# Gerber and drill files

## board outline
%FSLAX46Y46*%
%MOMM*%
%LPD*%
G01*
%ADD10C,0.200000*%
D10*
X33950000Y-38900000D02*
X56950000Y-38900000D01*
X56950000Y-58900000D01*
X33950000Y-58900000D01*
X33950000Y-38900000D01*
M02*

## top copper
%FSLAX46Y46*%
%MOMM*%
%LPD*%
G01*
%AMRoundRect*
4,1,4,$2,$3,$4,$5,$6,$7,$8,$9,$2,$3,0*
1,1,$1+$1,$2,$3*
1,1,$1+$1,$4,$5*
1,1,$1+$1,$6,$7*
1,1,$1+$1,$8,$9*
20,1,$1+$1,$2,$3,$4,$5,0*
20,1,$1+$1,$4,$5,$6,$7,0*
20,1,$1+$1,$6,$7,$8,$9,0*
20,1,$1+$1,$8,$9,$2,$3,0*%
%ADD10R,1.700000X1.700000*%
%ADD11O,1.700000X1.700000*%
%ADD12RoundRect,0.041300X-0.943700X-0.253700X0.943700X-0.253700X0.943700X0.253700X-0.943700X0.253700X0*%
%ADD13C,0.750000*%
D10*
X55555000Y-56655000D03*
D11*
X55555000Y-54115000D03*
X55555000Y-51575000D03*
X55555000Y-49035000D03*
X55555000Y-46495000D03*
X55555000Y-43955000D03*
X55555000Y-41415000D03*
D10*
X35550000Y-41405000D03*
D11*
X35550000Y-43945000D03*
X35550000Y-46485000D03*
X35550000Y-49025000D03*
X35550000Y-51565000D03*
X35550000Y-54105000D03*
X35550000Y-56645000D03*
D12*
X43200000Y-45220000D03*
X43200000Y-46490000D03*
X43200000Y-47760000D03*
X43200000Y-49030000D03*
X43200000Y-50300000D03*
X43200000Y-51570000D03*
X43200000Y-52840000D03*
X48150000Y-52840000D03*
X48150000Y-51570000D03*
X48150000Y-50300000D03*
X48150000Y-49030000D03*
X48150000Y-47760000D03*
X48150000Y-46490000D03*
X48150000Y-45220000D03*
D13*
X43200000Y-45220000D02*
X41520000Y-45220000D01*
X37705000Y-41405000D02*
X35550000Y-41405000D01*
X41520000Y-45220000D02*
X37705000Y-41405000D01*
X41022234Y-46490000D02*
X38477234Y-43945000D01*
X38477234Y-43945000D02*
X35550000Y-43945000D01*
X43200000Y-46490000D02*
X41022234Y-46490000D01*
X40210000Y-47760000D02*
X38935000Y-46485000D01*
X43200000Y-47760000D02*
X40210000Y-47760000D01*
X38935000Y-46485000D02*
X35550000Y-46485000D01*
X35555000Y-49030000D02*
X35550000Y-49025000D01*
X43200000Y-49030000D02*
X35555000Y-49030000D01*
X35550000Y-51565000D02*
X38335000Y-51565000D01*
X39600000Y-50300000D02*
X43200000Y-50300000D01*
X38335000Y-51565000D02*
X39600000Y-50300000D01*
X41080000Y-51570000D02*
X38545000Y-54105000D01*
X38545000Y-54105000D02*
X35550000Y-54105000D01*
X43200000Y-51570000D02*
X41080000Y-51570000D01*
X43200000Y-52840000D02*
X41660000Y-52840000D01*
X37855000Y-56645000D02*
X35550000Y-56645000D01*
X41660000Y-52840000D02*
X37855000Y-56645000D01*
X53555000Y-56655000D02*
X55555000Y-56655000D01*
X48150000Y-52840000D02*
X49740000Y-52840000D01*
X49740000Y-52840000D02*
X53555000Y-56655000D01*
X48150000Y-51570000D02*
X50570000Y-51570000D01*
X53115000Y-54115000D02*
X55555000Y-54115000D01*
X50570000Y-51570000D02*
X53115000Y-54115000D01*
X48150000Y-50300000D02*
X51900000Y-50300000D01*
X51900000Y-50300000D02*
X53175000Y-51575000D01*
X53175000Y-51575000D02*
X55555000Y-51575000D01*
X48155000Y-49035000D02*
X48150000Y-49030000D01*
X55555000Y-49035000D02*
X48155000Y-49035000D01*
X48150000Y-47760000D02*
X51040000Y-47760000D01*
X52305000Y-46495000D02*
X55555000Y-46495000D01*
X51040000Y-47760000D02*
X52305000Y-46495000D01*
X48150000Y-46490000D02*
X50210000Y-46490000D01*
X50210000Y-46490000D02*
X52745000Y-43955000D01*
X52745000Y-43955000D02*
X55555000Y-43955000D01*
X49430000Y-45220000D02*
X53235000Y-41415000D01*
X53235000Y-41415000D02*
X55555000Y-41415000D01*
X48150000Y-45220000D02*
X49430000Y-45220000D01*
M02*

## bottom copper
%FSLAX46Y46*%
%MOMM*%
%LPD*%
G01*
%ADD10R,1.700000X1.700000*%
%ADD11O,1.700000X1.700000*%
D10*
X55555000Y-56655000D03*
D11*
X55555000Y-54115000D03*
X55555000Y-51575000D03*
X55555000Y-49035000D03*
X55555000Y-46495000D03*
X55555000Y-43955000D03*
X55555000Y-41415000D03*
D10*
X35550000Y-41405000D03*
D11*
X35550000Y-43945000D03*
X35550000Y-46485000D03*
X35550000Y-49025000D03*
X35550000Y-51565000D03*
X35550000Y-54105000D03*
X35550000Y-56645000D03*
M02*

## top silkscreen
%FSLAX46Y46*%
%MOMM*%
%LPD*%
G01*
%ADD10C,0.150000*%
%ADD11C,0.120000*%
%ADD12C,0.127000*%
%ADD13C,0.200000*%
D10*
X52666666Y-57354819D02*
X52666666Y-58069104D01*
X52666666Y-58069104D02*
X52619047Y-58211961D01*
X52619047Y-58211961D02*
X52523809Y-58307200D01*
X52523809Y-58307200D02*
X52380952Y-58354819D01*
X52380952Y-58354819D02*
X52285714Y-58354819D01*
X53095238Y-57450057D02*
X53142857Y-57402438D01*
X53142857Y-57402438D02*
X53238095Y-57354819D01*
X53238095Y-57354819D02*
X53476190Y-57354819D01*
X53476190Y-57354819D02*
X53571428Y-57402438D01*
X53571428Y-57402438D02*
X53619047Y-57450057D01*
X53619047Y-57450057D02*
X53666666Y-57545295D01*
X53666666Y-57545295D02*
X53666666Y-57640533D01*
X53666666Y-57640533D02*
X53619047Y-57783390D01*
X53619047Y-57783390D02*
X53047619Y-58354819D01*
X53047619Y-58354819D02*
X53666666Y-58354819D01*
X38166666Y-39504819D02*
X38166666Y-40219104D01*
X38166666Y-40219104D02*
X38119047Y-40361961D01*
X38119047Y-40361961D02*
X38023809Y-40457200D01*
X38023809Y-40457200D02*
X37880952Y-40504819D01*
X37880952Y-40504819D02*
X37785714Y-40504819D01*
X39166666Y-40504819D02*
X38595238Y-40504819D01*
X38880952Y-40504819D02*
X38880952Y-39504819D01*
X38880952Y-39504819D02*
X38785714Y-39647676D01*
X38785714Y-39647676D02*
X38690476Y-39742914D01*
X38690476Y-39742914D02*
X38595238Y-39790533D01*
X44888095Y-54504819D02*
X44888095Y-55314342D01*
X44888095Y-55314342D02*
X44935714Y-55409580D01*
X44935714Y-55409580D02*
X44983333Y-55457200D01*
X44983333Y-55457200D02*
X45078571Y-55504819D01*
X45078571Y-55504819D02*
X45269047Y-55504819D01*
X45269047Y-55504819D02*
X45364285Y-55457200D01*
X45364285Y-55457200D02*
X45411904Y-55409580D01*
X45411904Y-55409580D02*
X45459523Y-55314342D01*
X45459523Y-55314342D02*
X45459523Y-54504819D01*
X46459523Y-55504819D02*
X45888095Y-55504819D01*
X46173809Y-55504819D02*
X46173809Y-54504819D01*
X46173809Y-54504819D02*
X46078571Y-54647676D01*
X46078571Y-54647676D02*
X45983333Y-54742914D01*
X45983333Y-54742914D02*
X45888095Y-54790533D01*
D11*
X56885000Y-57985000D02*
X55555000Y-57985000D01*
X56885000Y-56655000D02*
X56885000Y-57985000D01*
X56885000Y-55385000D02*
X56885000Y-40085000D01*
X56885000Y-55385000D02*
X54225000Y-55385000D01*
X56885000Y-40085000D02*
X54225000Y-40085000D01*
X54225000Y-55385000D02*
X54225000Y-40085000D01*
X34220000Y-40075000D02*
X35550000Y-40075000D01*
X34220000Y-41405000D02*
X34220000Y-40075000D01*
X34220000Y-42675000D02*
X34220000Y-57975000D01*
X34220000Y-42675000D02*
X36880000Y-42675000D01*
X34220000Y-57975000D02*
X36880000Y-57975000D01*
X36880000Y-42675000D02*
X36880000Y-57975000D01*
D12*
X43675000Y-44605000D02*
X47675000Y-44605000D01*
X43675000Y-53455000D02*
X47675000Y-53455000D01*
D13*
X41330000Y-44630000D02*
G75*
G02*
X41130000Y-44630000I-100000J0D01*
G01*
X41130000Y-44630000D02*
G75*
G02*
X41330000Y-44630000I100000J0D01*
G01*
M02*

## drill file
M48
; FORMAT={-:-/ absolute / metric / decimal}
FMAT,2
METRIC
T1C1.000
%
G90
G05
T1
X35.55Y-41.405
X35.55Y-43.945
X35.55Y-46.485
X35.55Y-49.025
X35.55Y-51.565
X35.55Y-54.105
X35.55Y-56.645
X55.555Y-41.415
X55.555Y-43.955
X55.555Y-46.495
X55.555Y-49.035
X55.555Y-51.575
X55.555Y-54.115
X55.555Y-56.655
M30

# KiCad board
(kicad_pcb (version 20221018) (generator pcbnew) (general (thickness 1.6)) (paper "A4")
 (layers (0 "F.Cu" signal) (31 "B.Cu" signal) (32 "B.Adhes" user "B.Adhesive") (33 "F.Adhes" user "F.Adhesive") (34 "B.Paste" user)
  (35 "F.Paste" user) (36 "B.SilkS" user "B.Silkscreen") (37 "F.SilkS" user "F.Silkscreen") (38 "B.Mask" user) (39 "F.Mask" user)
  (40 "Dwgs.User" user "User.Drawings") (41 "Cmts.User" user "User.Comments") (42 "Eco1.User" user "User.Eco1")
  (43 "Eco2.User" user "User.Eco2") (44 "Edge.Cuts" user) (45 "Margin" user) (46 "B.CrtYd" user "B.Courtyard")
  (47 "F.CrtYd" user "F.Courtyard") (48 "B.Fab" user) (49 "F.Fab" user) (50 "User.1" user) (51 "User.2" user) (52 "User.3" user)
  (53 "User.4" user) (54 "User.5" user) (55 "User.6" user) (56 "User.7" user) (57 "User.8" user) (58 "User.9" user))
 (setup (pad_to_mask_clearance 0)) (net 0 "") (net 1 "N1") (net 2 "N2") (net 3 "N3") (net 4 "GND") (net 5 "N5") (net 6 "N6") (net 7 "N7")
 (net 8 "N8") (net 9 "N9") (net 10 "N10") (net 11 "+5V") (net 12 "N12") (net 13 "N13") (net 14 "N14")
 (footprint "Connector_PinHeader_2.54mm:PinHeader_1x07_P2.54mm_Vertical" (layer "F.Cu") (at 55.555 56.655 180)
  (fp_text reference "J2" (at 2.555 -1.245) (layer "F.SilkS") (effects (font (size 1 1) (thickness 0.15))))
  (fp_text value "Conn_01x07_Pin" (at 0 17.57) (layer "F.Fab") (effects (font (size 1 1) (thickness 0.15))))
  (fp_line (start -1.33 -1.33) (end 0 -1.33) (stroke (width 0.12) (type solid)) (layer "F.SilkS"))
  (fp_line (start -1.33 0) (end -1.33 -1.33) (stroke (width 0.12) (type solid)) (layer "F.SilkS"))
  (fp_line (start -1.33 1.27) (end -1.33 16.57) (stroke (width 0.12) (type solid)) (layer "F.SilkS"))
  (fp_line (start -1.33 1.27) (end 1.33 1.27) (stroke (width 0.12) (type solid)) (layer "F.SilkS"))
  (fp_line (start -1.33 16.57) (end 1.33 16.57) (stroke (width 0.12) (type solid)) (layer "F.SilkS"))
  (fp_line (start 1.33 1.27) (end 1.33 16.57) (stroke (width 0.12) (type solid)) (layer "F.SilkS"))
  (pad "1" thru_hole rect (at 0 0 180) (size 1.7 1.7) (drill 1) (layers "*.Cu" "*.Mask") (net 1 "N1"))
  (pad "2" thru_hole oval (at 0 2.54 180) (size 1.7 1.7) (drill 1) (layers "*.Cu" "*.Mask") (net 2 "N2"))
  (pad "3" thru_hole oval (at 0 5.08 180) (size 1.7 1.7) (drill 1) (layers "*.Cu" "*.Mask") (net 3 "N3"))
  (pad "4" thru_hole oval (at 0 7.62 180) (size 1.7 1.7) (drill 1) (layers "*.Cu" "*.Mask") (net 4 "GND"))
  (pad "5" thru_hole oval (at 0 10.16 180) (size 1.7 1.7) (drill 1) (layers "*.Cu" "*.Mask") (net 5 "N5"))
  (pad "6" thru_hole oval (at 0 12.7 180) (size 1.7 1.7) (drill 1) (layers "*.Cu" "*.Mask") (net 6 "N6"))
  (pad "7" thru_hole oval (at 0 15.24 180) (size 1.7 1.7) (drill 1) (layers "*.Cu" "*.Mask") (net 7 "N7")))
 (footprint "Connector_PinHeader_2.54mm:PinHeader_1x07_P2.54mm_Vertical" (layer "F.Cu") (at 35.55 41.405)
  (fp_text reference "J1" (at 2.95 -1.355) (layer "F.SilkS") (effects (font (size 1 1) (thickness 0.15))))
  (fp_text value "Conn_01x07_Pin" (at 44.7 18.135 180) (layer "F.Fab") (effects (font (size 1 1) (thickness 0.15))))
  (fp_line (start -1.33 -1.33) (end 0 -1.33) (stroke (width 0.12) (type solid)) (layer "F.SilkS"))
  (fp_line (start -1.33 0) (end -1.33 -1.33) (stroke (width 0.12) (type solid)) (layer "F.SilkS"))
  (fp_line (start -1.33 1.27) (end -1.33 16.57) (stroke (width 0.12) (type solid)) (layer "F.SilkS"))
  (fp_line (start -1.33 1.27) (end 1.33 1.27) (stroke (width 0.12) (type solid)) (layer "F.SilkS"))
  (fp_line (start -1.33 16.57) (end 1.33 16.57) (stroke (width 0.12) (type solid)) (layer "F.SilkS"))
  (fp_line (start 1.33 1.27) (end 1.33 16.57) (stroke (width 0.12) (type solid)) (layer "F.SilkS"))
  (pad "1" thru_hole rect (at 0 0) (size 1.7 1.7) (drill 1) (layers "*.Cu" "*.Mask") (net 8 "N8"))
  (pad "2" thru_hole oval (at 0 2.54) (size 1.7 1.7) (drill 1) (layers "*.Cu" "*.Mask") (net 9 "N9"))
  (pad "3" thru_hole oval (at 0 5.08) (size 1.7 1.7) (drill 1) (layers "*.Cu" "*.Mask") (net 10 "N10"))
  (pad "4" thru_hole oval (at 0 7.62) (size 1.7 1.7) (drill 1) (layers "*.Cu" "*.Mask") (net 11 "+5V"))
  (pad "5" thru_hole oval (at 0 10.16) (size 1.7 1.7) (drill 1) (layers "*.Cu" "*.Mask") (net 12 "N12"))
  (pad "6" thru_hole oval (at 0 12.7) (size 1.7 1.7) (drill 1) (layers "*.Cu" "*.Mask") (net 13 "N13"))
  (pad "7" thru_hole oval (at 0 15.24) (size 1.7 1.7) (drill 1) (layers "*.Cu" "*.Mask") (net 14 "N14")))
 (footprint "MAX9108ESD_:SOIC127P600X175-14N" (layer "F.Cu") (at 45.675 49.03)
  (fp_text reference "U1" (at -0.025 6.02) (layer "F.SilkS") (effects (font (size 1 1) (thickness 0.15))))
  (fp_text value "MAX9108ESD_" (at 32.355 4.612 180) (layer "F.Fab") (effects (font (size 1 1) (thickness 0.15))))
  (fp_line (start -2 -4.425) (end 2 -4.425) (stroke (width 0.127) (type solid)) (layer "F.SilkS"))
  (fp_line (start -2 4.425) (end 2 4.425) (stroke (width 0.127) (type solid)) (layer "F.SilkS"))
  (fp_circle (center -4.445 -4.4) (end -4.345 -4.4) (stroke (width 0.2) (type solid)) (fill none) (layer "F.SilkS"))
  (pad "1" smd roundrect (at -2.475 -3.81) (size 1.97 0.59) (layers "F.Cu" "F.Paste" "F.Mask") (roundrect_rratio 0.07) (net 8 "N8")
   (solder_mask_margin 0.102))
  (pad "2" smd roundrect (at -2.475 -2.54) (size 1.97 0.59) (layers "F.Cu" "F.Paste" "F.Mask") (roundrect_rratio 0.07) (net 9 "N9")
   (solder_mask_margin 0.102))
  (pad "3" smd roundrect (at -2.475 -1.27) (size 1.97 0.59) (layers "F.Cu" "F.Paste" "F.Mask") (roundrect_rratio 0.07) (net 10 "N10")
   (solder_mask_margin 0.102))
  (pad "4" smd roundrect (at -2.475 0) (size 1.97 0.59) (layers "F.Cu" "F.Paste" "F.Mask") (roundrect_rratio 0.07) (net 11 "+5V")
   (solder_mask_margin 0.102))
  (pad "5" smd roundrect (at -2.475 1.27) (size 1.97 0.59) (layers "F.Cu" "F.Paste" "F.Mask") (roundrect_rratio 0.07) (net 12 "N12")
   (solder_mask_margin 0.102))
  (pad "6" smd roundrect (at -2.475 2.54) (size 1.97 0.59) (layers "F.Cu" "F.Paste" "F.Mask") (roundrect_rratio 0.07) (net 13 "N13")
   (solder_mask_margin 0.102))
  (pad "7" smd roundrect (at -2.475 3.81) (size 1.97 0.59) (layers "F.Cu" "F.Paste" "F.Mask") (roundrect_rratio 0.07) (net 14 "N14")
   (solder_mask_margin 0.102))
  (pad "8" smd roundrect (at 2.475 3.81) (size 1.97 0.59) (layers "F.Cu" "F.Paste" "F.Mask") (roundrect_rratio 0.07) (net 1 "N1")
   (solder_mask_margin 0.102))
  (pad "9" smd roundrect (at 2.475 2.54) (size 1.97 0.59) (layers "F.Cu" "F.Paste" "F.Mask") (roundrect_rratio 0.07) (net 2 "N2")
   (solder_mask_margin 0.102))
  (pad "10" smd roundrect (at 2.475 1.27) (size 1.97 0.59) (layers "F.Cu" "F.Paste" "F.Mask") (roundrect_rratio 0.07) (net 3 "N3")
   (solder_mask_margin 0.102))
  (pad "11" smd roundrect (at 2.475 0) (size 1.97 0.59) (layers "F.Cu" "F.Paste" "F.Mask") (roundrect_rratio 0.07) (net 4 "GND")
   (solder_mask_margin 0.102))
  (pad "12" smd roundrect (at 2.475 -1.27) (size 1.97 0.59) (layers "F.Cu" "F.Paste" "F.Mask") (roundrect_rratio 0.07) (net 5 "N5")
   (solder_mask_margin 0.102))
  (pad "13" smd roundrect (at 2.475 -2.54) (size 1.97 0.59) (layers "F.Cu" "F.Paste" "F.Mask") (roundrect_rratio 0.07) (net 6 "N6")
   (solder_mask_margin 0.102))
  (pad "14" smd roundrect (at 2.475 -3.81) (size 1.97 0.59) (layers "F.Cu" "F.Paste" "F.Mask") (roundrect_rratio 0.07) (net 7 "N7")
   (solder_mask_margin 0.102)))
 (gr_rect (start 33.95 38.9) (end 56.95 58.9) (stroke (width 0.2) (type default)) (fill none) (layer "Edge.Cuts"))
 (segment (start 43.2 45.22) (end 41.52 45.22) (width 0.75) (layer "F.Cu") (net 8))
 (segment (start 37.705 41.405) (end 35.55 41.405) (width 0.75) (layer "F.Cu") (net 8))
 (segment (start 41.52 45.22) (end 37.705 41.405) (width 0.75) (layer "F.Cu") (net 8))
 (segment (start 41.022234 46.49) (end 38.477234 43.945) (width 0.75) (layer "F.Cu") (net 9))
 (segment (start 38.477234 43.945) (end 35.55 43.945) (width 0.75) (layer "F.Cu") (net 9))
 (segment (start 43.2 46.49) (end 41.022234 46.49) (width 0.75) (layer "F.Cu") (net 9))
 (segment (start 40.21 47.76) (end 38.935 46.485) (width 0.75) (layer "F.Cu") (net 10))
 (segment (start 43.2 47.76) (end 40.21 47.76) (width 0.75) (layer "F.Cu") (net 10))
 (segment (start 38.935 46.485) (end 35.55 46.485) (width 0.75) (layer "F.Cu") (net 10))
 (segment (start 35.555 49.03) (end 35.55 49.025) (width 0.75) (layer "F.Cu") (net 11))
 (segment (start 43.2 49.03) (end 35.555 49.03) (width 0.75) (layer "F.Cu") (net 11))
 (segment (start 35.55 51.565) (end 38.335 51.565) (width 0.75) (layer "F.Cu") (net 12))
 (segment (start 39.6 50.3) (end 43.2 50.3) (width 0.75) (layer "F.Cu") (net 12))
 (segment (start 38.335 51.565) (end 39.6 50.3) (width 0.75) (layer "F.Cu") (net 12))
 (segment (start 41.08 51.57) (end 38.545 54.105) (width 0.75) (layer "F.Cu") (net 13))
 (segment (start 38.545 54.105) (end 35.55 54.105) (width 0.75) (layer "F.Cu") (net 13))
 (segment (start 43.2 51.57) (end 41.08 51.57) (width 0.75) (layer "F.Cu") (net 13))
 (segment (start 43.2 52.84) (end 41.66 52.84) (width 0.75) (layer "F.Cu") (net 14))
 (segment (start 37.855 56.645) (end 35.55 56.645) (width 0.75) (layer "F.Cu") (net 14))
 (segment (start 41.66 52.84) (end 37.855 56.645) (width 0.75) (layer "F.Cu") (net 14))
 (segment (start 53.555 56.655) (end 55.555 56.655) (width 0.75) (layer "F.Cu") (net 1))
 (segment (start 48.15 52.84) (end 49.74 52.84) (width 0.75) (layer "F.Cu") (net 1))
 (segment (start 49.74 52.84) (end 53.555 56.655) (width 0.75) (layer "F.Cu") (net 1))
 (segment (start 48.15 51.57) (end 50.57 51.57) (width 0.75) (layer "F.Cu") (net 2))
 (segment (start 53.115 54.115) (end 55.555 54.115) (width 0.75) (layer "F.Cu") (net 2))
 (segment (start 50.57 51.57) (end 53.115 54.115) (width 0.75) (layer "F.Cu") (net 2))
 (segment (start 48.15 50.3) (end 51.9 50.3) (width 0.75) (layer "F.Cu") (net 3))
 (segment (start 51.9 50.3) (end 53.175 51.575) (width 0.75) (layer "F.Cu") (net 3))
 (segment (start 53.175 51.575) (end 55.555 51.575) (width 0.75) (layer "F.Cu") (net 3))
 (segment (start 48.155 49.035) (end 48.15 49.03) (width 0.75) (layer "F.Cu") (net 4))
 (segment (start 55.555 49.035) (end 48.155 49.035) (width 0.75) (layer "F.Cu") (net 4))
 (segment (start 48.15 47.76) (end 51.04 47.76) (width 0.75) (layer "F.Cu") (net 5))
 (segment (start 52.305 46.495) (end 55.555 46.495) (width 0.75) (layer "F.Cu") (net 5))
 (segment (start 51.04 47.76) (end 52.305 46.495) (width 0.75) (layer "F.Cu") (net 5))
 (segment (start 48.15 46.49) (end 50.21 46.49) (width 0.75) (layer "F.Cu") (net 6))
 (segment (start 50.21 46.49) (end 52.745 43.955) (width 0.75) (layer "F.Cu") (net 6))
 (segment (start 52.745 43.955) (end 55.555 43.955) (width 0.75) (layer "F.Cu") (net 6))
 (segment (start 49.43 45.22) (end 53.235 41.415) (width 0.75) (layer "F.Cu") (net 7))
 (segment (start 53.235 41.415) (end 55.555 41.415) (width 0.75) (layer "F.Cu") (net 7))
 (segment (start 48.15 45.22) (end 49.43 45.22) (width 0.75) (layer "F.Cu") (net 7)))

